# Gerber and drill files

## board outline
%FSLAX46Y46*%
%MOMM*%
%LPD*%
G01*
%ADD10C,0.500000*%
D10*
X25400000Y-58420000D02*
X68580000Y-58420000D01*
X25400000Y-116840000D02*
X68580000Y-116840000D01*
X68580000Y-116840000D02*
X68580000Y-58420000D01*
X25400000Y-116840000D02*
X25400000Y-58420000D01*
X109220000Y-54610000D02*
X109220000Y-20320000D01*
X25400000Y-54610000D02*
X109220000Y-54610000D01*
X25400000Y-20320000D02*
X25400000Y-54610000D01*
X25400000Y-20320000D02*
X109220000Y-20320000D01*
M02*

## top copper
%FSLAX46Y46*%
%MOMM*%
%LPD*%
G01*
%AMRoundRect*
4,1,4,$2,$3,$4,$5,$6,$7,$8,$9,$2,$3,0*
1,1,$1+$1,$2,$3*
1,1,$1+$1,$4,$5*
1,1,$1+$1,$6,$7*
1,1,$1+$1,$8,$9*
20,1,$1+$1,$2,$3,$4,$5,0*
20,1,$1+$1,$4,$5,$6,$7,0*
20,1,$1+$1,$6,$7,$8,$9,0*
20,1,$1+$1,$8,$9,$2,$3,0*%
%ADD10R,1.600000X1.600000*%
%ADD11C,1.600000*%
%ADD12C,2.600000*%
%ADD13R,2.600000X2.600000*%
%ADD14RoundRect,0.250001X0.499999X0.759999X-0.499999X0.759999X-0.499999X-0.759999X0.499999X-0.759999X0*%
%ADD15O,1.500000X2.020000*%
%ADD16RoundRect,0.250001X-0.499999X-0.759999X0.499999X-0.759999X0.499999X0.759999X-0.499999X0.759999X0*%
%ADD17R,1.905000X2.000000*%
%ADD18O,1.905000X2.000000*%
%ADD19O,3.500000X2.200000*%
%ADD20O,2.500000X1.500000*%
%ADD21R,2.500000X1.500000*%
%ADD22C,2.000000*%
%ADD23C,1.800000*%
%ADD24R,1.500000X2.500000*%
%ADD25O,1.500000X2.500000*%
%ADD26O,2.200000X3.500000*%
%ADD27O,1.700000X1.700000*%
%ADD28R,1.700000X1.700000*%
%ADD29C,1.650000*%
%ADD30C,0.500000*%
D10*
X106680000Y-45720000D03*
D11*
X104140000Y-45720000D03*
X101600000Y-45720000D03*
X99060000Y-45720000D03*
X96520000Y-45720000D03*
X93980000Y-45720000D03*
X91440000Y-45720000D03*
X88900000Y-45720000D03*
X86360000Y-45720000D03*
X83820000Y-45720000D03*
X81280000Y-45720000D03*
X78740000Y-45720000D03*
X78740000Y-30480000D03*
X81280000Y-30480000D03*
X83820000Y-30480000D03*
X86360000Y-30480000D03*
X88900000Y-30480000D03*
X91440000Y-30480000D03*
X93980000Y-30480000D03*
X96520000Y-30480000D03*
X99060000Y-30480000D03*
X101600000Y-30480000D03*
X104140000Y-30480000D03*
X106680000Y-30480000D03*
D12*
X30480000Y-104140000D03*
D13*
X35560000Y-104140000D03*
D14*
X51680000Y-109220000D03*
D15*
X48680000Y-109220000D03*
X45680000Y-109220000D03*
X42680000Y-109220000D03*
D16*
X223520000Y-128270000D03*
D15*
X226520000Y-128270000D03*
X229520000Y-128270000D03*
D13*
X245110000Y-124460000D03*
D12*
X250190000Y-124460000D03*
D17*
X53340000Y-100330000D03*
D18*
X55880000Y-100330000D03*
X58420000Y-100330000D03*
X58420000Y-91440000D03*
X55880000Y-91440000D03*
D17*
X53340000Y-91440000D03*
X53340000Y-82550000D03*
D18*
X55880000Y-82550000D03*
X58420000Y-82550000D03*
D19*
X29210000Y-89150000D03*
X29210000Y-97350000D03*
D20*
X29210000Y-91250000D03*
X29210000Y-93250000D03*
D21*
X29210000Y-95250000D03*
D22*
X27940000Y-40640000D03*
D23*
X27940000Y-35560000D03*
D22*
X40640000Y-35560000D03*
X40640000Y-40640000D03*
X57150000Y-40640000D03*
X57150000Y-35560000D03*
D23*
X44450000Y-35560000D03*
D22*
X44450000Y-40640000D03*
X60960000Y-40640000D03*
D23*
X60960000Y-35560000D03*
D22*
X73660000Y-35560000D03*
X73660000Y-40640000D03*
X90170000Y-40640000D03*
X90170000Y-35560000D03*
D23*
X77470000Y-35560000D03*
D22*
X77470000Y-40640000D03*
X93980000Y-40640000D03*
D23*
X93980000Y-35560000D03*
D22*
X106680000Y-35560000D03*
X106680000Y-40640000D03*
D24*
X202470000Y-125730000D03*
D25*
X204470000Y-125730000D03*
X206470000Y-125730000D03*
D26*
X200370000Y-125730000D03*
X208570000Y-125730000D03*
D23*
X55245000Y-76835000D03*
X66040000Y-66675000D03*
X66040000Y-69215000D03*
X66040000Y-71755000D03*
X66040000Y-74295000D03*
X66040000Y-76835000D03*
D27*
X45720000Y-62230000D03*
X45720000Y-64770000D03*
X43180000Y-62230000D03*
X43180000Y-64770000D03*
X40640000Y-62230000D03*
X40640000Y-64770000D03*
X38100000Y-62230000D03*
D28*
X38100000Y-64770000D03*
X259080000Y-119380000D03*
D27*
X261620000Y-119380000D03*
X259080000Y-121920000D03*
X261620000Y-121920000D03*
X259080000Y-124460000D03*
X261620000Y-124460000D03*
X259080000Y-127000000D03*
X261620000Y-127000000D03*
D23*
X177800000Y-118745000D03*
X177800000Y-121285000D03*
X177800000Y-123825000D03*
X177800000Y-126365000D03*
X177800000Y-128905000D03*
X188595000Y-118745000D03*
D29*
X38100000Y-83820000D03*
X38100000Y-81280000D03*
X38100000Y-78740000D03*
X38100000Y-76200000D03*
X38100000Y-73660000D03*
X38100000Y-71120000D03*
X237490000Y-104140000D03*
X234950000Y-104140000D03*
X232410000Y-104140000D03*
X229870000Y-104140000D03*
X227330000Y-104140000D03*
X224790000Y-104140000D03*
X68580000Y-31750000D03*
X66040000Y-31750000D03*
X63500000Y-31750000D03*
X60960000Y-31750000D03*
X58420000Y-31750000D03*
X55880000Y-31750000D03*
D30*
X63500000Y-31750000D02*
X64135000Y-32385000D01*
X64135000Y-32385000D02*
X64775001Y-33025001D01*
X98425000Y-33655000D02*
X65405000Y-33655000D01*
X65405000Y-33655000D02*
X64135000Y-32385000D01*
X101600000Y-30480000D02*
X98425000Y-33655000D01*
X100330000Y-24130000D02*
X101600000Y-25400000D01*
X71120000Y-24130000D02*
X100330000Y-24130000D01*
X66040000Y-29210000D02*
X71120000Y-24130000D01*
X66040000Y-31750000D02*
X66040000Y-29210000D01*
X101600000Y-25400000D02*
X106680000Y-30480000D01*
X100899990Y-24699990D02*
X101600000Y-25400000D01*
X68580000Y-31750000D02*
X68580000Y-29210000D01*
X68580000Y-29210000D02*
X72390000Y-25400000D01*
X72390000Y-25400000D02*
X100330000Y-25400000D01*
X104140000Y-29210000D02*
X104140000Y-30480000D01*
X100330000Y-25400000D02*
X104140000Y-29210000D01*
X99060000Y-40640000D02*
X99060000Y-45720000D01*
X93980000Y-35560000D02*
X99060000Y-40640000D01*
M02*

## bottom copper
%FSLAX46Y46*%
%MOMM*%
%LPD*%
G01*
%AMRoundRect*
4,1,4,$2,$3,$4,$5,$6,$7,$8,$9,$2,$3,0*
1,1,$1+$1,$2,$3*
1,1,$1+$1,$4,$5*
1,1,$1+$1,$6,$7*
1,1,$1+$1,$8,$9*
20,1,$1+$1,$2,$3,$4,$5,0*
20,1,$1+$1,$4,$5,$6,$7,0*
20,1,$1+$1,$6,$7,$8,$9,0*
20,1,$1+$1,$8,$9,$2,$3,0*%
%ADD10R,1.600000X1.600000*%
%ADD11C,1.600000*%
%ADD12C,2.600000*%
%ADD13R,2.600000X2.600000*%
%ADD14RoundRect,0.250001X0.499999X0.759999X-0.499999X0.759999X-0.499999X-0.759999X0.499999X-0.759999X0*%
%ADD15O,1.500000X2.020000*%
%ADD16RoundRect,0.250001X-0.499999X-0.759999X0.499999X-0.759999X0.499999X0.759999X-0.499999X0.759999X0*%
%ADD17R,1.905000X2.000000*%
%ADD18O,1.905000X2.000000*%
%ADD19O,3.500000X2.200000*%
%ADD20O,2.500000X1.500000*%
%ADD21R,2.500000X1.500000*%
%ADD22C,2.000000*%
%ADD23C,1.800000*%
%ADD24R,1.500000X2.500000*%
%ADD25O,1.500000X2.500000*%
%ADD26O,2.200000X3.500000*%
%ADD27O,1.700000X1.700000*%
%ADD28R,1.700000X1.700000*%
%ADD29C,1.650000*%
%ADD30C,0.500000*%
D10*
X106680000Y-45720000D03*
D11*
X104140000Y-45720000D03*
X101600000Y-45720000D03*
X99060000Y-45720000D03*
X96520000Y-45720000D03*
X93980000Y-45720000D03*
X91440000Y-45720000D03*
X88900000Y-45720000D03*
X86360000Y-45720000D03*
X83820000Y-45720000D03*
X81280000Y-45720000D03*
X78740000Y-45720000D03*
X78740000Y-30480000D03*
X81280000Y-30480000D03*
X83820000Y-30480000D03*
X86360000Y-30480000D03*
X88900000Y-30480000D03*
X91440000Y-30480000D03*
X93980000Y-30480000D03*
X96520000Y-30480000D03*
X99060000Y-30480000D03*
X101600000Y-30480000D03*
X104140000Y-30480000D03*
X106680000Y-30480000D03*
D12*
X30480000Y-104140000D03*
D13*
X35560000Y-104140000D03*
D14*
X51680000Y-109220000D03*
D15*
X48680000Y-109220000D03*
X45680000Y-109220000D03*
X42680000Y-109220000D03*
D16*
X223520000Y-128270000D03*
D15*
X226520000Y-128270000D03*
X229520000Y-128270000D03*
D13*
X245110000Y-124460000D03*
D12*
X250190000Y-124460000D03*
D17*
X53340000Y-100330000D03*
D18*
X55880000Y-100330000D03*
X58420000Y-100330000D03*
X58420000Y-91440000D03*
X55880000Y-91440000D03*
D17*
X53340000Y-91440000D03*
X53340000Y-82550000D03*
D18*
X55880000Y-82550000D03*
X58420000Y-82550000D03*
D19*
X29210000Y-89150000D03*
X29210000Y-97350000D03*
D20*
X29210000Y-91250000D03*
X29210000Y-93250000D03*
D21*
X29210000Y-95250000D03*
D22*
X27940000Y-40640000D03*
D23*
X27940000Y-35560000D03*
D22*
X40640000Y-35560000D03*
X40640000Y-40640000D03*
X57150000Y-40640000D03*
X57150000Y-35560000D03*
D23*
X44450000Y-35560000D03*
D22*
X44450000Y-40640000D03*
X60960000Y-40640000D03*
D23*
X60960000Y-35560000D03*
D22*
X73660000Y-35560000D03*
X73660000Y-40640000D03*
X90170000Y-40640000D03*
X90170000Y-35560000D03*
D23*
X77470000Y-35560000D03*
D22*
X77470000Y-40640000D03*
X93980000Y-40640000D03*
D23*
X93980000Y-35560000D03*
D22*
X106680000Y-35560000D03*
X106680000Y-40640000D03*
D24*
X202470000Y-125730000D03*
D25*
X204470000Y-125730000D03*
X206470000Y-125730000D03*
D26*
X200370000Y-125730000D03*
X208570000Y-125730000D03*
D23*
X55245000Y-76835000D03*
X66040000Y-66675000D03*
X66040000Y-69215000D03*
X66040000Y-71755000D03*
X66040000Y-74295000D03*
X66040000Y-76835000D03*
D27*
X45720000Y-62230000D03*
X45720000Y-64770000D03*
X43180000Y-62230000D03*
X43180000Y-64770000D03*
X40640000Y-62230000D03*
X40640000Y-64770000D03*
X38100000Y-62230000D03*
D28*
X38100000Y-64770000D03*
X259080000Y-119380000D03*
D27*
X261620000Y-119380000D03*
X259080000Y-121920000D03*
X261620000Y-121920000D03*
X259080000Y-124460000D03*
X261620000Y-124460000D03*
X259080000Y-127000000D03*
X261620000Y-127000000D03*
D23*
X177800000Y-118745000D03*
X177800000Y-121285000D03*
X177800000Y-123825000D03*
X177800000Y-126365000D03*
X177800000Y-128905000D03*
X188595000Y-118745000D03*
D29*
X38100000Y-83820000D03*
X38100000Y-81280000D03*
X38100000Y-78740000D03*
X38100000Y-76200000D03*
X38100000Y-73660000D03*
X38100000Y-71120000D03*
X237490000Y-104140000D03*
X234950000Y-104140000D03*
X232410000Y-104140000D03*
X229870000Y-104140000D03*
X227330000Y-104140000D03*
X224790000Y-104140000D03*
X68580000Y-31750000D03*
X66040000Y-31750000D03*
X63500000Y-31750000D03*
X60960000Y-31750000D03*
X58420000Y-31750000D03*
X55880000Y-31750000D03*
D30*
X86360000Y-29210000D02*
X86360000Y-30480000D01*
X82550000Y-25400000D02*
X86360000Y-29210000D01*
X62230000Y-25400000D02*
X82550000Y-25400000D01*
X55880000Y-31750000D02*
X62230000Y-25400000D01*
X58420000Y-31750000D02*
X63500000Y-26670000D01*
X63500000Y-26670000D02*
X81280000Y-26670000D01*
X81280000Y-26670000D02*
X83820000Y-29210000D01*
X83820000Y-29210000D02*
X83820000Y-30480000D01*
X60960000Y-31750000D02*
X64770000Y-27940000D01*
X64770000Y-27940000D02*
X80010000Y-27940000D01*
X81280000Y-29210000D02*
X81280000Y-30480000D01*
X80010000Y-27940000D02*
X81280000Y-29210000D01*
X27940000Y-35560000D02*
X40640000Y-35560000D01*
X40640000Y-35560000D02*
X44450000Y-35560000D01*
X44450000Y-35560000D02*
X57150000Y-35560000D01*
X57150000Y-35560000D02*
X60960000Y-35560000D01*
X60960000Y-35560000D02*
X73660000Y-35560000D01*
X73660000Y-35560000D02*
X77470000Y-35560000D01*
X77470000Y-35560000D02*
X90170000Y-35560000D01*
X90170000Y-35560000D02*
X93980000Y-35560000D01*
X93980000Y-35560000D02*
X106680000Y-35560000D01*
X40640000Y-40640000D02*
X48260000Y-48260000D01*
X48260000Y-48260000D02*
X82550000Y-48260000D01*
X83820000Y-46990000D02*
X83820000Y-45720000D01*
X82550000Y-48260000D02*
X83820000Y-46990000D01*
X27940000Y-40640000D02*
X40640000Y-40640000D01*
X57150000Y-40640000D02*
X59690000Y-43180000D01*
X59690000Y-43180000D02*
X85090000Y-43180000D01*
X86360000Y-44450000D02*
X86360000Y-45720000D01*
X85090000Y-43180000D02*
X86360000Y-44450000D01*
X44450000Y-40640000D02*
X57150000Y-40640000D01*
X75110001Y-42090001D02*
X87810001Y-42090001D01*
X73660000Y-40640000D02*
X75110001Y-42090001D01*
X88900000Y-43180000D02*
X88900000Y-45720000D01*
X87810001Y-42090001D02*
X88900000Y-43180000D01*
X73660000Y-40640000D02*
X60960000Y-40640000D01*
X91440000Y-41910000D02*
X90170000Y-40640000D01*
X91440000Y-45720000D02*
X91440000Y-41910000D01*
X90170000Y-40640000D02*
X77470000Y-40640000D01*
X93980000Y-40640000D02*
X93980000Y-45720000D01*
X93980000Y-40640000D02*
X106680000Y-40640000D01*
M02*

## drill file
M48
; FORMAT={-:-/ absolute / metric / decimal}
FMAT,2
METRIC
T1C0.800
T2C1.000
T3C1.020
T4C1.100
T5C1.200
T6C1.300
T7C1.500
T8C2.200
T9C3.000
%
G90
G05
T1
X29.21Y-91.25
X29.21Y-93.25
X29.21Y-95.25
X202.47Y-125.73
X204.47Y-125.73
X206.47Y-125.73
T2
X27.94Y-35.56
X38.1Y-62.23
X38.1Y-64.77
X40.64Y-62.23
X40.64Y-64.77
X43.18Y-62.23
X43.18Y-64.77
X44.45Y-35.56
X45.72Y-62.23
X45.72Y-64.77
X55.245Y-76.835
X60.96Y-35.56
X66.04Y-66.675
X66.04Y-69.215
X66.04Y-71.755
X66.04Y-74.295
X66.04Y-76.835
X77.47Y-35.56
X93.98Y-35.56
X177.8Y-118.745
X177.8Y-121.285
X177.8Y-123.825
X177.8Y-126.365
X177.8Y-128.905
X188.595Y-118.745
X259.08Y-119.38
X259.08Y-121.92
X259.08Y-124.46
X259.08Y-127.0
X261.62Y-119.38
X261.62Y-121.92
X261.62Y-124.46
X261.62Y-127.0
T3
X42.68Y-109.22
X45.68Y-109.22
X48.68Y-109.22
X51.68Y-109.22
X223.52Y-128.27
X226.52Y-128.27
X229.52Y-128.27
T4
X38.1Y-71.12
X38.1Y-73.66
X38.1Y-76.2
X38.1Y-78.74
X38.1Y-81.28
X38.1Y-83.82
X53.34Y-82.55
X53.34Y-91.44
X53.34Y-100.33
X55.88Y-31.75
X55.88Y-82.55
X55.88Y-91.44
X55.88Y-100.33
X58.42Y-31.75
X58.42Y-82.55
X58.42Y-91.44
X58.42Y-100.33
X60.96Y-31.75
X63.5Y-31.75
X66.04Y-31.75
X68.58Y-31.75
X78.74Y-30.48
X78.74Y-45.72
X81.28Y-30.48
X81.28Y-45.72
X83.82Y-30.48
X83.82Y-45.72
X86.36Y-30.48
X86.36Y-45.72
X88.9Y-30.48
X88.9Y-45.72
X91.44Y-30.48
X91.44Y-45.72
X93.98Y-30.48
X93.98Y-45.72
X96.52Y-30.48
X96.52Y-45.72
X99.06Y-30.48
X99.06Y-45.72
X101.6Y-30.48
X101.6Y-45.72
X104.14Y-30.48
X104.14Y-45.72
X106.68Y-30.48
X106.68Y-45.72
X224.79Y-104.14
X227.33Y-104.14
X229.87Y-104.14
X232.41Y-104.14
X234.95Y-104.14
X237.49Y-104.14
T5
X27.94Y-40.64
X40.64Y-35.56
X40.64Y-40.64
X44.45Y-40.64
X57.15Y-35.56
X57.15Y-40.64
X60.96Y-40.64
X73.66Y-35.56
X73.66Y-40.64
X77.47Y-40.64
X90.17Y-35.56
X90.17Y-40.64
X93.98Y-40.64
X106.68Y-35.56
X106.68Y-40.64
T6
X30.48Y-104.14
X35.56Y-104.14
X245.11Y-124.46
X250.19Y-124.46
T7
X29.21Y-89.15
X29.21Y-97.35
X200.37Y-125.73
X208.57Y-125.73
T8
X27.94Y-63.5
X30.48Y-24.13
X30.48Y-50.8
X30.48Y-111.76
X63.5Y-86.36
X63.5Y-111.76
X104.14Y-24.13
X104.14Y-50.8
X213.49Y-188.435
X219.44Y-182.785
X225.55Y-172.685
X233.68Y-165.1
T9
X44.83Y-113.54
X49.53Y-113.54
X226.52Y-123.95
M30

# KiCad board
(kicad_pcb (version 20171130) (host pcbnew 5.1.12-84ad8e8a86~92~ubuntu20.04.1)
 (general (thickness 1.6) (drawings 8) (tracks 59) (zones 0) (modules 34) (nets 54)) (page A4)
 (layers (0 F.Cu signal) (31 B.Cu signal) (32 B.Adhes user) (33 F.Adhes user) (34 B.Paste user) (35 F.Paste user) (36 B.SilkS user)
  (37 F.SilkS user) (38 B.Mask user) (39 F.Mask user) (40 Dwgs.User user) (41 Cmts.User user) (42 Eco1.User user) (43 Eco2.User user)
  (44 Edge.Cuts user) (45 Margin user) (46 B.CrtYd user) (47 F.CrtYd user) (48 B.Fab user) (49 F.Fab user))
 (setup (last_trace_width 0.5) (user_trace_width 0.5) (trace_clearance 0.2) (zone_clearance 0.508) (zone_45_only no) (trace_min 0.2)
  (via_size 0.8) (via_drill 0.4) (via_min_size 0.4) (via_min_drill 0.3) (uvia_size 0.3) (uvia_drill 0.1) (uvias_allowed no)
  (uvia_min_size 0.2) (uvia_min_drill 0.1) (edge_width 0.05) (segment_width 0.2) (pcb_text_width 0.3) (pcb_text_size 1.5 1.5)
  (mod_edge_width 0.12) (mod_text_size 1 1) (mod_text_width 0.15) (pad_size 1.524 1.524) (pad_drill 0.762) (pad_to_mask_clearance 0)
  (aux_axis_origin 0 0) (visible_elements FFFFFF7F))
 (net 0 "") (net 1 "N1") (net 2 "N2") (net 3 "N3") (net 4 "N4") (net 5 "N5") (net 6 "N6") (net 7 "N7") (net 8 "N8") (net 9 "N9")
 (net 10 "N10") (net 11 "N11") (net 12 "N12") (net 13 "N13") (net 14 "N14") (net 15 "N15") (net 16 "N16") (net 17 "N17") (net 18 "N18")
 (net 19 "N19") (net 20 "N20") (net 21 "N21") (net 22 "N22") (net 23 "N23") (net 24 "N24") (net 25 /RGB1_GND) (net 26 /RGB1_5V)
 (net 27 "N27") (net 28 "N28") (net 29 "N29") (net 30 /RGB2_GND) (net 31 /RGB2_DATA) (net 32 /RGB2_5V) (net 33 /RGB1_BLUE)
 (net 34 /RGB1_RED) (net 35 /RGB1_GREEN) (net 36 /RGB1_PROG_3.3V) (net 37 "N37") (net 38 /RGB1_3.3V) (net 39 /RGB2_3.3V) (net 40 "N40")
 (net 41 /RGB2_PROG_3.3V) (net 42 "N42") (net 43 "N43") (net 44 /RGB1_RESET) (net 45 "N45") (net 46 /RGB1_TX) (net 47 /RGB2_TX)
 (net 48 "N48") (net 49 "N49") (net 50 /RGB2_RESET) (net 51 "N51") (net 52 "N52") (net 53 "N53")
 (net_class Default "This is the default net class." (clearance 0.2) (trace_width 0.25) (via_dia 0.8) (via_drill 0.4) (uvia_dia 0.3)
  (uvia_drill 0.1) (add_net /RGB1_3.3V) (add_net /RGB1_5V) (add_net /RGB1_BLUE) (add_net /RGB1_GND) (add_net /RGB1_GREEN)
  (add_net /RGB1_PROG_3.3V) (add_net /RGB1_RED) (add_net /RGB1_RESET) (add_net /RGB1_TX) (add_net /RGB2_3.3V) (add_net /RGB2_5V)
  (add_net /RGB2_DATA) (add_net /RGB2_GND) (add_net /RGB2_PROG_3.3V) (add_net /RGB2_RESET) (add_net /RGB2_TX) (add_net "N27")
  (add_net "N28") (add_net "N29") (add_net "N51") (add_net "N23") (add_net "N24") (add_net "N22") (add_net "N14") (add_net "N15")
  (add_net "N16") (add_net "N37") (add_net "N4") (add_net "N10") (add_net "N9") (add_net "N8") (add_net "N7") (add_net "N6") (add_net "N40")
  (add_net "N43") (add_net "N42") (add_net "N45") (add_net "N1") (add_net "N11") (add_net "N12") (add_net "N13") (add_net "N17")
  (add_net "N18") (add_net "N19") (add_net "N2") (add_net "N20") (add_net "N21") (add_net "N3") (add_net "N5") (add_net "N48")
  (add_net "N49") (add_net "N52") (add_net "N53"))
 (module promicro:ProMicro (layer B.Cu) (at 106.68 45.72 180)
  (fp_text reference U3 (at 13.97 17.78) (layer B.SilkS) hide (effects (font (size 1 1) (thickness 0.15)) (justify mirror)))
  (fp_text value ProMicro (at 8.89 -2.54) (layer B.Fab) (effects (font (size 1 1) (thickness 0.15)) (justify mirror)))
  (pad 1 thru_hole rect (at 0 0 180) (size 1.6 1.6) (drill 1.1) (layers *.Cu *.Mask B.SilkS) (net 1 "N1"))
  (pad 2 thru_hole circle (at 2.54 0 180) (size 1.6 1.6) (drill 1.1) (layers *.Cu *.Mask B.SilkS) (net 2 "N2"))
  (pad 3 thru_hole circle (at 5.08 0 180) (size 1.6 1.6) (drill 1.1) (layers *.Cu *.Mask B.SilkS) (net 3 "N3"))
  (pad 4 thru_hole circle (at 7.62 0 180) (size 1.6 1.6) (drill 1.1) (layers *.Cu *.Mask B.SilkS) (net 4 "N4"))
  (pad 5 thru_hole circle (at 10.16 0 180) (size 1.6 1.6) (drill 1.1) (layers *.Cu *.Mask B.SilkS) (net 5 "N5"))
  (pad 6 thru_hole circle (at 12.7 0 180) (size 1.6 1.6) (drill 1.1) (layers *.Cu *.Mask B.SilkS) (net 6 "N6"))
  (pad 7 thru_hole circle (at 15.24 0 180) (size 1.6 1.6) (drill 1.1) (layers *.Cu *.Mask B.SilkS) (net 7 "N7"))
  (pad 8 thru_hole circle (at 17.78 0 180) (size 1.6 1.6) (drill 1.1) (layers *.Cu *.Mask B.SilkS) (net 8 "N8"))
  (pad 9 thru_hole circle (at 20.32 0 180) (size 1.6 1.6) (drill 1.1) (layers *.Cu *.Mask B.SilkS) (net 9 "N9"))
  (pad 10 thru_hole circle (at 22.86 0 180) (size 1.6 1.6) (drill 1.1) (layers *.Cu *.Mask B.SilkS) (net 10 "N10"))
  (pad 11 thru_hole circle (at 25.4 0 180) (size 1.6 1.6) (drill 1.1) (layers *.Cu *.Mask B.SilkS) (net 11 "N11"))
  (pad 12 thru_hole circle (at 27.94 0 180) (size 1.6 1.6) (drill 1.1) (layers *.Cu *.Mask B.SilkS) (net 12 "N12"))
  (pad 13 thru_hole circle (at 27.94 15.24 180) (size 1.6 1.6) (drill 1.1) (layers *.Cu *.Mask B.SilkS) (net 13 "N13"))
  (pad 14 thru_hole circle (at 25.4 15.24 180) (size 1.6 1.6) (drill 1.1) (layers *.Cu *.Mask B.SilkS) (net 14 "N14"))
  (pad 15 thru_hole circle (at 22.86 15.24 180) (size 1.6 1.6) (drill 1.1) (layers *.Cu *.Mask B.SilkS) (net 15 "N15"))
  (pad 16 thru_hole circle (at 20.32 15.24 180) (size 1.6 1.6) (drill 1.1) (layers *.Cu *.Mask B.SilkS) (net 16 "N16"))
  (pad 17 thru_hole circle (at 17.78 15.24 180) (size 1.6 1.6) (drill 1.1) (layers *.Cu *.Mask B.SilkS) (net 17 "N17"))
  (pad 18 thru_hole circle (at 15.24 15.24 180) (size 1.6 1.6) (drill 1.1) (layers *.Cu *.Mask B.SilkS) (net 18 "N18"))
  (pad 19 thru_hole circle (at 12.7 15.24 180) (size 1.6 1.6) (drill 1.1) (layers *.Cu *.Mask B.SilkS) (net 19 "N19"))
  (pad 20 thru_hole circle (at 10.16 15.24 180) (size 1.6 1.6) (drill 1.1) (layers *.Cu *.Mask B.SilkS) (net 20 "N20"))
  (pad 21 thru_hole circle (at 7.62 15.24 180) (size 1.6 1.6) (drill 1.1) (layers *.Cu *.Mask B.SilkS) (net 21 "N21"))
  (pad 22 thru_hole circle (at 5.08 15.24 180) (size 1.6 1.6) (drill 1.1) (layers *.Cu *.Mask B.SilkS) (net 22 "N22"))
  (pad 23 thru_hole circle (at 2.54 15.24 180) (size 1.6 1.6) (drill 1.1) (layers *.Cu *.Mask B.SilkS) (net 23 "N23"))
  (pad 24 thru_hole circle (at 0 15.24 180) (size 1.6 1.6) (drill 1.1) (layers *.Cu *.Mask B.SilkS) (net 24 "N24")))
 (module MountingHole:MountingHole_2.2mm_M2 (layer F.Cu) (at 27.94 63.5)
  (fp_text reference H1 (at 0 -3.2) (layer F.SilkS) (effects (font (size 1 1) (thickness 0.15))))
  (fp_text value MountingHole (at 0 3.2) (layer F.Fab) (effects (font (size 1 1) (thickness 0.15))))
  (pad 1 np_thru_hole circle (at 0 0) (size 2.2 2.2) (drill 2.2) (layers *.Cu *.Mask)))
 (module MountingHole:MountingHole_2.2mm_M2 (layer F.Cu) (at 30.48 111.76)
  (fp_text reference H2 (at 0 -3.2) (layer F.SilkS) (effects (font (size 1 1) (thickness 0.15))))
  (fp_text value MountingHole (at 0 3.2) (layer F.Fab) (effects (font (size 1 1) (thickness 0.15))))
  (pad 1 np_thru_hole circle (at 0 0) (size 2.2 2.2) (drill 2.2) (layers *.Cu *.Mask)))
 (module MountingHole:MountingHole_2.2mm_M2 (layer F.Cu) (at 63.5 111.76)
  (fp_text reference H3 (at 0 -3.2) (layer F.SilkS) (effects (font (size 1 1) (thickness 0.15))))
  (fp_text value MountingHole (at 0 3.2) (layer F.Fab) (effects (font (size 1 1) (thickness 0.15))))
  (pad 1 np_thru_hole circle (at 0 0) (size 2.2 2.2) (drill 2.2) (layers *.Cu *.Mask)))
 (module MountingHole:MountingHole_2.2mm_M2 (layer F.Cu) (at 63.5 86.36)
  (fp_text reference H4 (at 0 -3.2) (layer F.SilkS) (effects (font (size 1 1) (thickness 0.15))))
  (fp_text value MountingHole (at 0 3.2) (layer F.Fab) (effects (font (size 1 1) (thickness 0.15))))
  (pad 1 np_thru_hole circle (at 0 0) (size 2.2 2.2) (drill 2.2) (layers *.Cu *.Mask)))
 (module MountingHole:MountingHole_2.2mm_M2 (layer F.Cu) (at 233.68 165.1)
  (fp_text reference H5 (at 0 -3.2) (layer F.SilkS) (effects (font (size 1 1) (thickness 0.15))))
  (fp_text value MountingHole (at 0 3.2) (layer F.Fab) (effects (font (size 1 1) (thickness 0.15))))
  (pad 1 np_thru_hole circle (at 0 0) (size 2.2 2.2) (drill 2.2) (layers *.Cu *.Mask)))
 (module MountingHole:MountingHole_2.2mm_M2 (layer F.Cu) (at 219.440001 182.785001)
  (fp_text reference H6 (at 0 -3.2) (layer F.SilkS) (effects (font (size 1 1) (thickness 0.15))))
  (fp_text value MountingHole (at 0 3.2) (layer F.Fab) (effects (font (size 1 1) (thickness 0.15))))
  (pad 1 np_thru_hole circle (at 0 0) (size 2.2 2.2) (drill 2.2) (layers *.Cu *.Mask)))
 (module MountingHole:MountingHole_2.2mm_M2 (layer F.Cu) (at 225.550001 172.685001)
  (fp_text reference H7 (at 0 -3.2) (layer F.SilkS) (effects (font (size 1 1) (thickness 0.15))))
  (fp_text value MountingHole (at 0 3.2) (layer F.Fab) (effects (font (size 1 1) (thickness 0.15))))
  (pad 1 np_thru_hole circle (at 0 0) (size 2.2 2.2) (drill 2.2) (layers *.Cu *.Mask)))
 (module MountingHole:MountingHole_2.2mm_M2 (layer F.Cu) (at 213.490001 188.435001)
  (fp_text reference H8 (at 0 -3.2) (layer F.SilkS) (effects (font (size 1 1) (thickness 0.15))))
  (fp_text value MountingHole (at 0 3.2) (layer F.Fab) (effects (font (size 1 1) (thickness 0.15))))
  (pad 1 np_thru_hole circle (at 0 0) (size 2.2 2.2) (drill 2.2) (layers *.Cu *.Mask)))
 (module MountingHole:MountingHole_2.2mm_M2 (layer F.Cu) (at 30.48 50.8)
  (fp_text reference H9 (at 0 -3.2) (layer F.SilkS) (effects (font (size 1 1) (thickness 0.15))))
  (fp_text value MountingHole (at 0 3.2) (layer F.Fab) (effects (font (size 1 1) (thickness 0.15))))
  (pad 1 np_thru_hole circle (at 0 0) (size 2.2 2.2) (drill 2.2) (layers *.Cu *.Mask)))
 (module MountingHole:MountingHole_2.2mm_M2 (layer F.Cu) (at 104.14 50.8)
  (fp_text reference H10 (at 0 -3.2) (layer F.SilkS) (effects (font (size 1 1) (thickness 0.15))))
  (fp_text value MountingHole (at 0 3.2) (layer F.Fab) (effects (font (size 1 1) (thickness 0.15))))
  (pad 1 np_thru_hole circle (at 0 0) (size 2.2 2.2) (drill 2.2) (layers *.Cu *.Mask)))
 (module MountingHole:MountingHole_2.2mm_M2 (layer F.Cu) (at 104.14 24.13)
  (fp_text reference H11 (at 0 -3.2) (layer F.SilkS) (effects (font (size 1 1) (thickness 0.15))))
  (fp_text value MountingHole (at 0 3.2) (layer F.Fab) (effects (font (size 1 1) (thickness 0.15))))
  (pad 1 np_thru_hole circle (at 0 0) (size 2.2 2.2) (drill 2.2) (layers *.Cu *.Mask)))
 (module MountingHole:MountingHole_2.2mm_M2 (layer F.Cu) (at 30.48 24.13)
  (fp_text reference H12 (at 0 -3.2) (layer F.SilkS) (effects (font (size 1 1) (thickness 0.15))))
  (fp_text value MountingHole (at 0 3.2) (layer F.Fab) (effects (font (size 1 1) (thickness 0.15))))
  (pad 1 np_thru_hole circle (at 0 0) (size 2.2 2.2) (drill 2.2) (layers *.Cu *.Mask)))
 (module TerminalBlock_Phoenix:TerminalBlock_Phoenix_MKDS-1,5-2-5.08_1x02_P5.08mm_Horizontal (layer F.Cu) (at 35.56 104.14 180)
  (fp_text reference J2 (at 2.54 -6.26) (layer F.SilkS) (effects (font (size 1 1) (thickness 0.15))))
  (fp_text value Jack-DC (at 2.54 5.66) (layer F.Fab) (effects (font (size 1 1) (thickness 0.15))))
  (pad 2 thru_hole circle (at 5.08 0 180) (size 2.6 2.6) (drill 1.3) (layers *.Cu *.Mask) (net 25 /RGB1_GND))
  (pad 1 thru_hole rect (at 0 0 180) (size 2.6 2.6) (drill 1.3) (layers *.Cu *.Mask) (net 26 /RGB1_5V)))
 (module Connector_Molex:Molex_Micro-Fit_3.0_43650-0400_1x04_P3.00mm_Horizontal (layer F.Cu) (at 51.68 109.22 180)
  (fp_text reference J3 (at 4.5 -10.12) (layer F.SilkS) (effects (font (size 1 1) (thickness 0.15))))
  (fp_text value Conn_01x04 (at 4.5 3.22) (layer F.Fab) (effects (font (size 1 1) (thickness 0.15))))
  (pad "" np_thru_hole circle (at 2.15 -4.32 180) (size 3 3) (drill 3) (layers *.Cu *.Mask))
  (pad "" np_thru_hole circle (at 6.85 -4.32 180) (size 3 3) (drill 3) (layers *.Cu *.Mask))
  (pad 1 thru_hole roundrect (at 0 0 180) (size 1.5 2.02) (drill 1.02) (layers *.Cu *.Mask) (roundrect_rratio 0.166667) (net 26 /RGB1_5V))
  (pad 2 thru_hole oval (at 3 0 180) (size 1.5 2.02) (drill 1.02) (layers *.Cu *.Mask) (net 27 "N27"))
  (pad 3 thru_hole oval (at 6 0 180) (size 1.5 2.02) (drill 1.02) (layers *.Cu *.Mask) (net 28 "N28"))
  (pad 4 thru_hole oval (at 9 0 180) (size 1.5 2.02) (drill 1.02) (layers *.Cu *.Mask) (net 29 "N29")))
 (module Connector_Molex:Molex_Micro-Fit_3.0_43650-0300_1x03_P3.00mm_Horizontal (layer F.Cu) (at 223.52 128.27)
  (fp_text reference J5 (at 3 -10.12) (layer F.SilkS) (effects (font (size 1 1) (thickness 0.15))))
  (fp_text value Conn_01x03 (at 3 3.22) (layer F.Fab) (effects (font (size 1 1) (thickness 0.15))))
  (pad "" np_thru_hole circle (at 3 -4.32) (size 3 3) (drill 3) (layers *.Cu *.Mask))
  (pad 1 thru_hole roundrect (at 0 0) (size 1.5 2.02) (drill 1.02) (layers *.Cu *.Mask) (roundrect_rratio 0.166667) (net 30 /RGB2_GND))
  (pad 2 thru_hole oval (at 3 0) (size 1.5 2.02) (drill 1.02) (layers *.Cu *.Mask) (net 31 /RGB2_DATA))
  (pad 3 thru_hole oval (at 6 0) (size 1.5 2.02) (drill 1.02) (layers *.Cu *.Mask) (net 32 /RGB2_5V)))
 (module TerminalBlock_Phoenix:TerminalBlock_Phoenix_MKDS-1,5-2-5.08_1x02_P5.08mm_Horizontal (layer F.Cu) (at 245.11 124.46)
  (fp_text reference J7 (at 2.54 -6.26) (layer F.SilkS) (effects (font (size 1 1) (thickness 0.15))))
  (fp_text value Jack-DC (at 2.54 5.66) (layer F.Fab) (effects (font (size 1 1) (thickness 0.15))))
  (pad 1 thru_hole rect (at 0 0) (size 2.6 2.6) (drill 1.3) (layers *.Cu *.Mask) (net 32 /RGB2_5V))
  (pad 2 thru_hole circle (at 5.08 0) (size 2.6 2.6) (drill 1.3) (layers *.Cu *.Mask) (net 30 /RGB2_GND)))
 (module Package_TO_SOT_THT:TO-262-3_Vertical (layer F.Cu) (at 53.34 100.33)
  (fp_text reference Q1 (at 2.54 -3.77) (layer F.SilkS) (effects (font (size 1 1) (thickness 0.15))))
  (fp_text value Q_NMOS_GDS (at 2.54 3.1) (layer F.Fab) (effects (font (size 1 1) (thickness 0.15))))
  (pad 1 thru_hole rect (at 0 0) (size 1.905 2) (drill 1.1) (layers *.Cu *.Mask) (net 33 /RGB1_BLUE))
  (pad 2 thru_hole oval (at 2.54 0) (size 1.905 2) (drill 1.1) (layers *.Cu *.Mask) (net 27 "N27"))
  (pad 3 thru_hole oval (at 5.08 0) (size 1.905 2) (drill 1.1) (layers *.Cu *.Mask) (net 25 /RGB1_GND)))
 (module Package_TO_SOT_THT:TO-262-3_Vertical (layer F.Cu) (at 53.34 91.44)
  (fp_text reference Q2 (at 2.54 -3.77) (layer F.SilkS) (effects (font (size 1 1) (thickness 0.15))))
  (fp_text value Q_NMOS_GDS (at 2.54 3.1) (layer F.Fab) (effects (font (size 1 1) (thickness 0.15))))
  (pad 3 thru_hole oval (at 5.08 0) (size 1.905 2) (drill 1.1) (layers *.Cu *.Mask) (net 25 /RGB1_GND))
  (pad 2 thru_hole oval (at 2.54 0) (size 1.905 2) (drill 1.1) (layers *.Cu *.Mask) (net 28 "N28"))
  (pad 1 thru_hole rect (at 0 0) (size 1.905 2) (drill 1.1) (layers *.Cu *.Mask) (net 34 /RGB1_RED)))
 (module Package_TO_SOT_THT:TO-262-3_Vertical (layer F.Cu) (at 53.34 82.55)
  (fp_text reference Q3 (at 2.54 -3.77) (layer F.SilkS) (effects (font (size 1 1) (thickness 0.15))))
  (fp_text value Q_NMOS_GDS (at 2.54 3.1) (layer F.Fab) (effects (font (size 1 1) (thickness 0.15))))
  (pad 1 thru_hole rect (at 0 0) (size 1.905 2) (drill 1.1) (layers *.Cu *.Mask) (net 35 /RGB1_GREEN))
  (pad 2 thru_hole oval (at 2.54 0) (size 1.905 2) (drill 1.1) (layers *.Cu *.Mask) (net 29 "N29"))
  (pad 3 thru_hole oval (at 5.08 0) (size 1.905 2) (drill 1.1) (layers *.Cu *.Mask) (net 25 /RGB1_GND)))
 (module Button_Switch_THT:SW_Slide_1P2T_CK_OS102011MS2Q (layer F.Cu) (at 29.21 95.25 90)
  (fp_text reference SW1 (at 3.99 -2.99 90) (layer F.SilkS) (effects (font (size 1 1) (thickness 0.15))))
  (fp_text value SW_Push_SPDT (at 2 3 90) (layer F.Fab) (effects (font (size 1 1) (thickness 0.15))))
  (pad "" thru_hole oval (at 6.1 0 90) (size 2.2 3.5) (drill 1.5) (layers *.Cu *.Mask))
  (pad "" thru_hole oval (at -2.1 0 90) (size 2.2 3.5) (drill 1.5) (layers *.Cu *.Mask))
  (pad 3 thru_hole oval (at 4 0 90) (size 1.5 2.5) (drill 0.8) (layers *.Cu *.Mask) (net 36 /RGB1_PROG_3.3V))
  (pad 2 thru_hole oval (at 2 0 90) (size 1.5 2.5) (drill 0.8) (layers *.Cu *.Mask) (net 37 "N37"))
  (pad 1 thru_hole rect (at 0 0 90) (size 1.5 2.5) (drill 0.8) (layers *.Cu *.Mask) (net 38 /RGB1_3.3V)))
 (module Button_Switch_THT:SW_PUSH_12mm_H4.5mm (layer F.Cu) (at 33.02 38.1 180)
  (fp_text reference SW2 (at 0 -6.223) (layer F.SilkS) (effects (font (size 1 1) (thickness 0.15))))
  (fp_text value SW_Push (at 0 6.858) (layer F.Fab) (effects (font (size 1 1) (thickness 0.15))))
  (pad 2 thru_hole circle (at 5.08 -2.54 180) (size 2 2) (drill 1.2) (layers *.Cu *.Mask) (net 10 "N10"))
  (pad 1 thru_hole circle (at 5.08 2.54 180) (size 1.8 1.8) (drill 1) (layers *.Cu *.Mask) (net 4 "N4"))
  (pad 1 thru_hole circle (at -7.62 2.54 180) (size 2 2) (drill 1.2) (layers *.Cu *.Mask) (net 4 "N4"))
  (pad 2 thru_hole circle (at -7.62 -2.54 180) (size 2 2) (drill 1.2) (layers *.Cu *.Mask) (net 10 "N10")))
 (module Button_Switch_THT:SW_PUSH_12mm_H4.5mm (layer F.Cu) (at 49.53 38.1 180)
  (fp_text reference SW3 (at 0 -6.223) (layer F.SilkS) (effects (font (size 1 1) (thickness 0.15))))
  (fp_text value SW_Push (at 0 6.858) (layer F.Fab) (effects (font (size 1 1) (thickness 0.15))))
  (pad 2 thru_hole circle (at -7.62 -2.54 180) (size 2 2) (drill 1.2) (layers *.Cu *.Mask) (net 9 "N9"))
  (pad 1 thru_hole circle (at -7.62 2.54 180) (size 2 2) (drill 1.2) (layers *.Cu *.Mask) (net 4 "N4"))
  (pad 1 thru_hole circle (at 5.08 2.54 180) (size 1.8 1.8) (drill 1) (layers *.Cu *.Mask) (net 4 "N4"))
  (pad 2 thru_hole circle (at 5.08 -2.54 180) (size 2 2) (drill 1.2) (layers *.Cu *.Mask) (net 9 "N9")))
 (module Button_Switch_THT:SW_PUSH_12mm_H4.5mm (layer F.Cu) (at 66.04 38.1 180)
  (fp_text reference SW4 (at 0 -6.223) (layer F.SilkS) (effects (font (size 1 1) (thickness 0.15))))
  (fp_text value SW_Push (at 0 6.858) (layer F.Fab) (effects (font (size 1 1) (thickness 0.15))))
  (pad 2 thru_hole circle (at 5.08 -2.54 180) (size 2 2) (drill 1.2) (layers *.Cu *.Mask) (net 8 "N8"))
  (pad 1 thru_hole circle (at 5.08 2.54 180) (size 1.8 1.8) (drill 1) (layers *.Cu *.Mask) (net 4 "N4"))
  (pad 1 thru_hole circle (at -7.62 2.54 180) (size 2 2) (drill 1.2) (layers *.Cu *.Mask) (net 4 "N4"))
  (pad 2 thru_hole circle (at -7.62 -2.54 180) (size 2 2) (drill 1.2) (layers *.Cu *.Mask) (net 8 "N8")))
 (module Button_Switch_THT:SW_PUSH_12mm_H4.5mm (layer F.Cu) (at 82.55 38.1 180)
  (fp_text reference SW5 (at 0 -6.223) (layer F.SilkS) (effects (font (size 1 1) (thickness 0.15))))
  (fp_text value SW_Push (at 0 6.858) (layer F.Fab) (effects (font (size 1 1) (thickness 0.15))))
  (pad 2 thru_hole circle (at -7.62 -2.54 180) (size 2 2) (drill 1.2) (layers *.Cu *.Mask) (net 7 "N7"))
  (pad 1 thru_hole circle (at -7.62 2.54 180) (size 2 2) (drill 1.2) (layers *.Cu *.Mask) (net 4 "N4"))
  (pad 1 thru_hole circle (at 5.08 2.54 180) (size 1.8 1.8) (drill 1) (layers *.Cu *.Mask) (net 4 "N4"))
  (pad 2 thru_hole circle (at 5.08 -2.54 180) (size 2 2) (drill 1.2) (layers *.Cu *.Mask) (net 7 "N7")))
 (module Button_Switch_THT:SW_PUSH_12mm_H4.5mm (layer F.Cu) (at 99.06 38.1 180)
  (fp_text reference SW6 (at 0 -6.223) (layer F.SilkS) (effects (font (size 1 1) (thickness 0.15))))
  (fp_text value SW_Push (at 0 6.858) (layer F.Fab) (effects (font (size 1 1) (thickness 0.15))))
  (pad 2 thru_hole circle (at 5.08 -2.54 180) (size 2 2) (drill 1.2) (layers *.Cu *.Mask) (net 6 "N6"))
  (pad 1 thru_hole circle (at 5.08 2.54 180) (size 1.8 1.8) (drill 1) (layers *.Cu *.Mask) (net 4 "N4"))
  (pad 1 thru_hole circle (at -7.62 2.54 180) (size 2 2) (drill 1.2) (layers *.Cu *.Mask) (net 4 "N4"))
  (pad 2 thru_hole circle (at -7.62 -2.54 180) (size 2 2) (drill 1.2) (layers *.Cu *.Mask) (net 6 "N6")))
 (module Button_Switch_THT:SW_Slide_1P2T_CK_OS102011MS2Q (layer F.Cu) (at 202.47 125.73)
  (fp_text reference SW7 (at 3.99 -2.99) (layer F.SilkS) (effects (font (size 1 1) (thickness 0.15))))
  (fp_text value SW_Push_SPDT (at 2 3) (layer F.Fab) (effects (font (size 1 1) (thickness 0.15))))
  (pad 1 thru_hole rect (at 0 0) (size 1.5 2.5) (drill 0.8) (layers *.Cu *.Mask) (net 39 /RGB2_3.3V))
  (pad 2 thru_hole oval (at 2 0) (size 1.5 2.5) (drill 0.8) (layers *.Cu *.Mask) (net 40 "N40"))
  (pad 3 thru_hole oval (at 4 0) (size 1.5 2.5) (drill 0.8) (layers *.Cu *.Mask) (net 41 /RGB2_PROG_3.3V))
  (pad "" thru_hole oval (at -2.1 0) (size 2.2 3.5) (drill 1.5) (layers *.Cu *.Mask))
  (pad "" thru_hole oval (at 6.1 0) (size 2.2 3.5) (drill 1.5) (layers *.Cu *.Mask)))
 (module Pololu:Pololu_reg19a (layer F.Cu) (at 58.42 69.85 180)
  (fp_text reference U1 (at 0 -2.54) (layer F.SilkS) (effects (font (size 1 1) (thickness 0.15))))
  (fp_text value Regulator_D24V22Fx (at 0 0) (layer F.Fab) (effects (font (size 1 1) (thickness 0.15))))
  (pad 6 thru_hole circle (at 3.175 -6.985 180) (size 1.8 1.8) (drill 1) (layers *.Cu *.Mask) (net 25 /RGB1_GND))
  (pad 5 thru_hole circle (at -7.62 3.175 180) (size 1.8 1.8) (drill 1) (layers *.Cu *.Mask) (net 38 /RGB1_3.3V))
  (pad 4 thru_hole circle (at -7.62 0.635 180) (size 1.8 1.8) (drill 1) (layers *.Cu *.Mask) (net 25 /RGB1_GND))
  (pad 3 thru_hole circle (at -7.62 -1.905 180) (size 1.8 1.8) (drill 1) (layers *.Cu *.Mask) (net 26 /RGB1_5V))
  (pad 2 thru_hole circle (at -7.62 -4.445 180) (size 1.8 1.8) (drill 1) (layers *.Cu *.Mask) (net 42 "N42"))
  (pad 1 thru_hole circle (at -7.62 -6.985 180) (size 1.8 1.8) (drill 1) (layers *.Cu *.Mask) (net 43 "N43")))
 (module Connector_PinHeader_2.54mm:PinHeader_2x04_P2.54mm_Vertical (layer F.Cu) (at 38.1 64.77 90)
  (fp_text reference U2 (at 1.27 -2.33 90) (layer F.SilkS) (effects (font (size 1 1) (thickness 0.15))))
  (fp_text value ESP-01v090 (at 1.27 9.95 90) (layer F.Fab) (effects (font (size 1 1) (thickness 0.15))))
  (pad 8 thru_hole oval (at 2.54 7.62 90) (size 1.7 1.7) (drill 1) (layers *.Cu *.Mask) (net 35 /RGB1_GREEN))
  (pad 7 thru_hole oval (at 0 7.62 90) (size 1.7 1.7) (drill 1) (layers *.Cu *.Mask) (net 37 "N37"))
  (pad 6 thru_hole oval (at 2.54 5.08 90) (size 1.7 1.7) (drill 1) (layers *.Cu *.Mask) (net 34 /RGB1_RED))
  (pad 5 thru_hole oval (at 0 5.08 90) (size 1.7 1.7) (drill 1) (layers *.Cu *.Mask) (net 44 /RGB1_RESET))
  (pad 4 thru_hole oval (at 2.54 2.54 90) (size 1.7 1.7) (drill 1) (layers *.Cu *.Mask) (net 33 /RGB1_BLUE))
  (pad 3 thru_hole oval (at 0 2.54 90) (size 1.7 1.7) (drill 1) (layers *.Cu *.Mask) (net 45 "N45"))
  (pad 2 thru_hole oval (at 2.54 0 90) (size 1.7 1.7) (drill 1) (layers *.Cu *.Mask) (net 25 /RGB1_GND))
  (pad 1 thru_hole rect (at 0 0 90) (size 1.7 1.7) (drill 1) (layers *.Cu *.Mask) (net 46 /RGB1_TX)))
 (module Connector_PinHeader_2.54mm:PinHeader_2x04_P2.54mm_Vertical (layer F.Cu) (at 259.08 119.38)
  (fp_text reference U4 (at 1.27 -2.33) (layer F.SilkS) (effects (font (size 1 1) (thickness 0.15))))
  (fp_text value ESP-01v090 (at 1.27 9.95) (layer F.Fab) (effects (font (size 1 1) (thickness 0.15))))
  (pad 1 thru_hole rect (at 0 0) (size 1.7 1.7) (drill 1) (layers *.Cu *.Mask) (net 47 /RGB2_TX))
  (pad 2 thru_hole oval (at 2.54 0) (size 1.7 1.7) (drill 1) (layers *.Cu *.Mask) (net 30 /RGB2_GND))
  (pad 3 thru_hole oval (at 0 2.54) (size 1.7 1.7) (drill 1) (layers *.Cu *.Mask) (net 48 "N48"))
  (pad 4 thru_hole oval (at 2.54 2.54) (size 1.7 1.7) (drill 1) (layers *.Cu *.Mask) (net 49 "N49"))
  (pad 5 thru_hole oval (at 0 5.08) (size 1.7 1.7) (drill 1) (layers *.Cu *.Mask) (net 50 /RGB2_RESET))
  (pad 6 thru_hole oval (at 2.54 5.08) (size 1.7 1.7) (drill 1) (layers *.Cu *.Mask) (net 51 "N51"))
  (pad 7 thru_hole oval (at 0 7.62) (size 1.7 1.7) (drill 1) (layers *.Cu *.Mask) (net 40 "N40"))
  (pad 8 thru_hole oval (at 2.54 7.62) (size 1.7 1.7) (drill 1) (layers *.Cu *.Mask) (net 31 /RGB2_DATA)))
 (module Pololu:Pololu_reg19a (layer F.Cu) (at 185.42 125.73)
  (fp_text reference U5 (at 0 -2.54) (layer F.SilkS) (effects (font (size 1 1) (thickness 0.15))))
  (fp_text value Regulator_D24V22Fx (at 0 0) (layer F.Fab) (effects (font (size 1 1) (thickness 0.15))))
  (pad 1 thru_hole circle (at -7.62 -6.985) (size 1.8 1.8) (drill 1) (layers *.Cu *.Mask) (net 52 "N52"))
  (pad 2 thru_hole circle (at -7.62 -4.445) (size 1.8 1.8) (drill 1) (layers *.Cu *.Mask) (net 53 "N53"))
  (pad 3 thru_hole circle (at -7.62 -1.905) (size 1.8 1.8) (drill 1) (layers *.Cu *.Mask) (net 32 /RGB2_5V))
  (pad 4 thru_hole circle (at -7.62 0.635) (size 1.8 1.8) (drill 1) (layers *.Cu *.Mask) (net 30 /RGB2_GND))
  (pad 5 thru_hole circle (at -7.62 3.175) (size 1.8 1.8) (drill 1) (layers *.Cu *.Mask) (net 39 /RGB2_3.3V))
  (pad 6 thru_hole circle (at 3.175 -6.985) (size 1.8 1.8) (drill 1) (layers *.Cu *.Mask) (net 30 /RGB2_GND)))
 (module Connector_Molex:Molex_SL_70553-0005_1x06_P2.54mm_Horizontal (layer B.Cu) (at 38.1 71.12 90)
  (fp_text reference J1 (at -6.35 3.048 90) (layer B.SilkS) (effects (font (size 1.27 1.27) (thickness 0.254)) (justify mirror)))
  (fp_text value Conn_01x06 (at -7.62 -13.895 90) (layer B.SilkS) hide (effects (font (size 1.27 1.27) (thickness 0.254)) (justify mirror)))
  (pad 6 thru_hole circle (at -12.7 0 90) (size 1.65 1.65) (drill 1.1) (layers *.Cu *.Mask) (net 44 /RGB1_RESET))
  (pad 5 thru_hole circle (at -10.16 0 90) (size 1.65 1.65) (drill 1.1) (layers *.Cu *.Mask) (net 34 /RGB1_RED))
  (pad 4 thru_hole circle (at -7.62 0 90) (size 1.65 1.65) (drill 1.1) (layers *.Cu *.Mask) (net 35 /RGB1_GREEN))
  (pad 3 thru_hole circle (at -5.08 0 90) (size 1.65 1.65) (drill 1.1) (layers *.Cu *.Mask) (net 46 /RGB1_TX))
  (pad 2 thru_hole circle (at -2.54 0 90) (size 1.65 1.65) (drill 1.1) (layers *.Cu *.Mask) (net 36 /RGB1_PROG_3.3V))
  (pad 1 thru_hole circle (at 0 0 90) (size 1.65 1.65) (drill 1.1) (layers *.Cu *.Mask) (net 25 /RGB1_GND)))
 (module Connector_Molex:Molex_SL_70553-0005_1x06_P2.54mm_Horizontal (layer F.Cu) (at 237.49 104.14)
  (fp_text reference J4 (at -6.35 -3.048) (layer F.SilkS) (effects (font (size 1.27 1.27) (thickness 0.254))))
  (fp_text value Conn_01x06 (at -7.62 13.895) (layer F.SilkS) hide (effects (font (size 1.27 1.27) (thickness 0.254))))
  (pad 1 thru_hole circle (at 0 0) (size 1.65 1.65) (drill 1.1) (layers *.Cu *.Mask) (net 30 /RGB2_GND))
  (pad 2 thru_hole circle (at -2.54 0) (size 1.65 1.65) (drill 1.1) (layers *.Cu *.Mask) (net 41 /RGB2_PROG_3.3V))
  (pad 3 thru_hole circle (at -5.08 0) (size 1.65 1.65) (drill 1.1) (layers *.Cu *.Mask) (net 47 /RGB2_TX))
  (pad 4 thru_hole circle (at -7.62 0) (size 1.65 1.65) (drill 1.1) (layers *.Cu *.Mask) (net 31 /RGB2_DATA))
  (pad 5 thru_hole circle (at -10.16 0) (size 1.65 1.65) (drill 1.1) (layers *.Cu *.Mask) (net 51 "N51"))
  (pad 6 thru_hole circle (at -12.7 0) (size 1.65 1.65) (drill 1.1) (layers *.Cu *.Mask) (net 50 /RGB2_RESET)))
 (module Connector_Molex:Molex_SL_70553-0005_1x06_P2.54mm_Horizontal (layer B.Cu) (at 68.58 31.75)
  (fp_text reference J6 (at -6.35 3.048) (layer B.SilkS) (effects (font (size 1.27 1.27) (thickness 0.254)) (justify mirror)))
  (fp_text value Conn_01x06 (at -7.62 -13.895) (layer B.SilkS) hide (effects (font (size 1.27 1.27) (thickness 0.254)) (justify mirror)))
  (pad 1 thru_hole circle (at 0 0) (size 1.65 1.65) (drill 1.1) (layers *.Cu *.Mask) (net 23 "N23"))
  (pad 2 thru_hole circle (at -2.54 0) (size 1.65 1.65) (drill 1.1) (layers *.Cu *.Mask) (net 24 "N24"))
  (pad 3 thru_hole circle (at -5.08 0) (size 1.65 1.65) (drill 1.1) (layers *.Cu *.Mask) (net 22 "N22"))
  (pad 4 thru_hole circle (at -7.62 0) (size 1.65 1.65) (drill 1.1) (layers *.Cu *.Mask) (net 14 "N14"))
  (pad 5 thru_hole circle (at -10.16 0) (size 1.65 1.65) (drill 1.1) (layers *.Cu *.Mask) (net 15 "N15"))
  (pad 6 thru_hole circle (at -12.7 0) (size 1.65 1.65) (drill 1.1) (layers *.Cu *.Mask) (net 16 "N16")))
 (gr_line (start 25.4 58.42) (end 68.58 58.42) (layer Edge.Cuts) (width 0.5))
 (gr_line (start 25.4 116.84) (end 68.58 116.84) (layer Edge.Cuts) (width 0.5))
 (gr_line (start 68.58 116.84) (end 68.58 58.42) (layer Edge.Cuts) (width 0.5))
 (gr_line (start 25.4 116.84) (end 25.4 58.42) (layer Edge.Cuts) (width 0.5))
 (gr_line (start 109.22 54.61) (end 109.22 20.32) (layer Edge.Cuts) (width 0.5))
 (gr_line (start 25.4 54.61) (end 109.22 54.61) (layer Edge.Cuts) (width 0.5))
 (gr_line (start 25.4 20.32) (end 25.4 54.61) (layer Edge.Cuts) (width 0.5))
 (gr_line (start 25.4 20.32) (end 109.22 20.32) (layer Edge.Cuts) (width 0.5))
 (segment (start 86.36 29.21) (end 86.36 30.48) (width 0.5) (layer B.Cu) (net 16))
 (segment (start 82.55 25.4) (end 86.36 29.21) (width 0.5) (layer B.Cu) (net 16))
 (segment (start 62.23 25.4) (end 82.55 25.4) (width 0.5) (layer B.Cu) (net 16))
 (segment (start 55.88 31.75) (end 62.23 25.4) (width 0.5) (layer B.Cu) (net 16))
 (segment (start 58.42 31.75) (end 63.5 26.67) (width 0.5) (layer B.Cu) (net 15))
 (segment (start 63.5 26.67) (end 81.28 26.67) (width 0.5) (layer B.Cu) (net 15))
 (segment (start 81.28 26.67) (end 83.82 29.21) (width 0.5) (layer B.Cu) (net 15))
 (segment (start 83.82 29.21) (end 83.82 30.48) (width 0.5) (layer B.Cu) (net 15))
 (segment (start 60.96 31.75) (end 64.77 27.94) (width 0.5) (layer B.Cu) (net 14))
 (segment (start 64.77 27.94) (end 80.01 27.94) (width 0.5) (layer B.Cu) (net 14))
 (segment (start 81.28 29.21) (end 81.28 30.48) (width 0.5) (layer B.Cu) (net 14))
 (segment (start 80.01 27.94) (end 81.28 29.21) (width 0.5) (layer B.Cu) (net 14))
 (segment (start 63.5 31.75) (end 64.135 32.385) (width 0.5) (layer F.Cu) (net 22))
 (segment (start 64.135 32.385) (end 64.775001 33.025001) (width 0.5) (layer F.Cu) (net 22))
 (segment (start 98.425 33.655) (end 65.405 33.655) (width 0.5) (layer F.Cu) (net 22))
 (segment (start 65.405 33.655) (end 64.135 32.385) (width 0.5) (layer F.Cu) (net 22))
 (segment (start 101.6 30.48) (end 98.425 33.655) (width 0.5) (layer F.Cu) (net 22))
 (segment (start 100.33 24.13) (end 101.6 25.4) (width 0.5) (layer F.Cu) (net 24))
 (segment (start 71.12 24.13) (end 100.33 24.13) (width 0.5) (layer F.Cu) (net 24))
 (segment (start 66.04 29.21) (end 71.12 24.13) (width 0.5) (layer F.Cu) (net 24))
 (segment (start 66.04 31.75) (end 66.04 29.21) (width 0.5) (layer F.Cu) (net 24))
 (segment (start 101.6 25.4) (end 106.68 30.48) (width 0.5) (layer F.Cu) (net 24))
 (segment (start 100.89999 24.69999) (end 101.6 25.4) (width 0.5) (layer F.Cu) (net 24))
 (segment (start 68.58 31.75) (end 68.58 29.21) (width 0.5) (layer F.Cu) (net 23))
 (segment (start 68.58 29.21) (end 72.39 25.4) (width 0.5) (layer F.Cu) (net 23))
 (segment (start 72.39 25.4) (end 100.33 25.4) (width 0.5) (layer F.Cu) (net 23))
 (segment (start 104.14 29.21) (end 104.14 30.48) (width 0.5) (layer F.Cu) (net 23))
 (segment (start 100.33 25.4) (end 104.14 29.21) (width 0.5) (layer F.Cu) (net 23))
 (segment (start 27.94 35.56) (end 40.64 35.56) (width 0.5) (layer B.Cu) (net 4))
 (segment (start 40.64 35.56) (end 44.45 35.56) (width 0.5) (layer B.Cu) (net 4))
 (segment (start 44.45 35.56) (end 57.15 35.56) (width 0.5) (layer B.Cu) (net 4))
 (segment (start 57.15 35.56) (end 60.96 35.56) (width 0.5) (layer B.Cu) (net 4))
 (segment (start 60.96 35.56) (end 73.66 35.56) (width 0.5) (layer B.Cu) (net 4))
 (segment (start 73.66 35.56) (end 77.47 35.56) (width 0.5) (layer B.Cu) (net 4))
 (segment (start 77.47 35.56) (end 90.17 35.56) (width 0.5) (layer B.Cu) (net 4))
 (segment (start 90.17 35.56) (end 93.98 35.56) (width 0.5) (layer B.Cu) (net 4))
 (segment (start 93.98 35.56) (end 106.68 35.56) (width 0.5) (layer B.Cu) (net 4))
 (segment (start 99.06 40.64) (end 99.06 45.72) (width 0.5) (layer F.Cu) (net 4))
 (segment (start 93.98 35.56) (end 99.06 40.64) (width 0.5) (layer F.Cu) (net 4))
 (segment (start 40.64 40.64) (end 48.26 48.26) (width 0.5) (layer B.Cu) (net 10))
 (segment (start 48.26 48.26) (end 82.55 48.26) (width 0.5) (layer B.Cu) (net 10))
 (segment (start 83.82 46.99) (end 83.82 45.72) (width 0.5) (layer B.Cu) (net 10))
 (segment (start 82.55 48.26) (end 83.82 46.99) (width 0.5) (layer B.Cu) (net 10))
 (segment (start 27.94 40.64) (end 40.64 40.64) (width 0.5) (layer B.Cu) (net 10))
 (segment (start 57.15 40.64) (end 59.69 43.18) (width 0.5) (layer B.Cu) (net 9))
 (segment (start 59.69 43.18) (end 85.09 43.18) (width 0.5) (layer B.Cu) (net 9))
 (segment (start 86.36 44.45) (end 86.36 45.72) (width 0.5) (layer B.Cu) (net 9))
 (segment (start 85.09 43.18) (end 86.36 44.45) (width 0.5) (layer B.Cu) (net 9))
 (segment (start 44.45 40.64) (end 57.15 40.64) (width 0.5) (layer B.Cu) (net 9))
 (segment (start 75.110001 42.090001) (end 87.810001 42.090001) (width 0.5) (layer B.Cu) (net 8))
 (segment (start 73.66 40.64) (end 75.110001 42.090001) (width 0.5) (layer B.Cu) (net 8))
 (segment (start 88.9 43.18) (end 88.9 45.72) (width 0.5) (layer B.Cu) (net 8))
 (segment (start 87.810001 42.090001) (end 88.9 43.18) (width 0.5) (layer B.Cu) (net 8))
 (segment (start 73.66 40.64) (end 60.96 40.64) (width 0.5) (layer B.Cu) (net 8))
 (segment (start 91.44 41.91) (end 90.17 40.64) (width 0.5) (layer B.Cu) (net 7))
 (segment (start 91.44 45.72) (end 91.44 41.91) (width 0.5) (layer B.Cu) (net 7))
 (segment (start 90.17 40.64) (end 77.47 40.64) (width 0.5) (layer B.Cu) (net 7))
 (segment (start 93.98 40.64) (end 93.98 45.72) (width 0.5) (layer B.Cu) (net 6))
 (segment (start 93.98 40.64) (end 106.68 40.64) (width 0.5) (layer B.Cu) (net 6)))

